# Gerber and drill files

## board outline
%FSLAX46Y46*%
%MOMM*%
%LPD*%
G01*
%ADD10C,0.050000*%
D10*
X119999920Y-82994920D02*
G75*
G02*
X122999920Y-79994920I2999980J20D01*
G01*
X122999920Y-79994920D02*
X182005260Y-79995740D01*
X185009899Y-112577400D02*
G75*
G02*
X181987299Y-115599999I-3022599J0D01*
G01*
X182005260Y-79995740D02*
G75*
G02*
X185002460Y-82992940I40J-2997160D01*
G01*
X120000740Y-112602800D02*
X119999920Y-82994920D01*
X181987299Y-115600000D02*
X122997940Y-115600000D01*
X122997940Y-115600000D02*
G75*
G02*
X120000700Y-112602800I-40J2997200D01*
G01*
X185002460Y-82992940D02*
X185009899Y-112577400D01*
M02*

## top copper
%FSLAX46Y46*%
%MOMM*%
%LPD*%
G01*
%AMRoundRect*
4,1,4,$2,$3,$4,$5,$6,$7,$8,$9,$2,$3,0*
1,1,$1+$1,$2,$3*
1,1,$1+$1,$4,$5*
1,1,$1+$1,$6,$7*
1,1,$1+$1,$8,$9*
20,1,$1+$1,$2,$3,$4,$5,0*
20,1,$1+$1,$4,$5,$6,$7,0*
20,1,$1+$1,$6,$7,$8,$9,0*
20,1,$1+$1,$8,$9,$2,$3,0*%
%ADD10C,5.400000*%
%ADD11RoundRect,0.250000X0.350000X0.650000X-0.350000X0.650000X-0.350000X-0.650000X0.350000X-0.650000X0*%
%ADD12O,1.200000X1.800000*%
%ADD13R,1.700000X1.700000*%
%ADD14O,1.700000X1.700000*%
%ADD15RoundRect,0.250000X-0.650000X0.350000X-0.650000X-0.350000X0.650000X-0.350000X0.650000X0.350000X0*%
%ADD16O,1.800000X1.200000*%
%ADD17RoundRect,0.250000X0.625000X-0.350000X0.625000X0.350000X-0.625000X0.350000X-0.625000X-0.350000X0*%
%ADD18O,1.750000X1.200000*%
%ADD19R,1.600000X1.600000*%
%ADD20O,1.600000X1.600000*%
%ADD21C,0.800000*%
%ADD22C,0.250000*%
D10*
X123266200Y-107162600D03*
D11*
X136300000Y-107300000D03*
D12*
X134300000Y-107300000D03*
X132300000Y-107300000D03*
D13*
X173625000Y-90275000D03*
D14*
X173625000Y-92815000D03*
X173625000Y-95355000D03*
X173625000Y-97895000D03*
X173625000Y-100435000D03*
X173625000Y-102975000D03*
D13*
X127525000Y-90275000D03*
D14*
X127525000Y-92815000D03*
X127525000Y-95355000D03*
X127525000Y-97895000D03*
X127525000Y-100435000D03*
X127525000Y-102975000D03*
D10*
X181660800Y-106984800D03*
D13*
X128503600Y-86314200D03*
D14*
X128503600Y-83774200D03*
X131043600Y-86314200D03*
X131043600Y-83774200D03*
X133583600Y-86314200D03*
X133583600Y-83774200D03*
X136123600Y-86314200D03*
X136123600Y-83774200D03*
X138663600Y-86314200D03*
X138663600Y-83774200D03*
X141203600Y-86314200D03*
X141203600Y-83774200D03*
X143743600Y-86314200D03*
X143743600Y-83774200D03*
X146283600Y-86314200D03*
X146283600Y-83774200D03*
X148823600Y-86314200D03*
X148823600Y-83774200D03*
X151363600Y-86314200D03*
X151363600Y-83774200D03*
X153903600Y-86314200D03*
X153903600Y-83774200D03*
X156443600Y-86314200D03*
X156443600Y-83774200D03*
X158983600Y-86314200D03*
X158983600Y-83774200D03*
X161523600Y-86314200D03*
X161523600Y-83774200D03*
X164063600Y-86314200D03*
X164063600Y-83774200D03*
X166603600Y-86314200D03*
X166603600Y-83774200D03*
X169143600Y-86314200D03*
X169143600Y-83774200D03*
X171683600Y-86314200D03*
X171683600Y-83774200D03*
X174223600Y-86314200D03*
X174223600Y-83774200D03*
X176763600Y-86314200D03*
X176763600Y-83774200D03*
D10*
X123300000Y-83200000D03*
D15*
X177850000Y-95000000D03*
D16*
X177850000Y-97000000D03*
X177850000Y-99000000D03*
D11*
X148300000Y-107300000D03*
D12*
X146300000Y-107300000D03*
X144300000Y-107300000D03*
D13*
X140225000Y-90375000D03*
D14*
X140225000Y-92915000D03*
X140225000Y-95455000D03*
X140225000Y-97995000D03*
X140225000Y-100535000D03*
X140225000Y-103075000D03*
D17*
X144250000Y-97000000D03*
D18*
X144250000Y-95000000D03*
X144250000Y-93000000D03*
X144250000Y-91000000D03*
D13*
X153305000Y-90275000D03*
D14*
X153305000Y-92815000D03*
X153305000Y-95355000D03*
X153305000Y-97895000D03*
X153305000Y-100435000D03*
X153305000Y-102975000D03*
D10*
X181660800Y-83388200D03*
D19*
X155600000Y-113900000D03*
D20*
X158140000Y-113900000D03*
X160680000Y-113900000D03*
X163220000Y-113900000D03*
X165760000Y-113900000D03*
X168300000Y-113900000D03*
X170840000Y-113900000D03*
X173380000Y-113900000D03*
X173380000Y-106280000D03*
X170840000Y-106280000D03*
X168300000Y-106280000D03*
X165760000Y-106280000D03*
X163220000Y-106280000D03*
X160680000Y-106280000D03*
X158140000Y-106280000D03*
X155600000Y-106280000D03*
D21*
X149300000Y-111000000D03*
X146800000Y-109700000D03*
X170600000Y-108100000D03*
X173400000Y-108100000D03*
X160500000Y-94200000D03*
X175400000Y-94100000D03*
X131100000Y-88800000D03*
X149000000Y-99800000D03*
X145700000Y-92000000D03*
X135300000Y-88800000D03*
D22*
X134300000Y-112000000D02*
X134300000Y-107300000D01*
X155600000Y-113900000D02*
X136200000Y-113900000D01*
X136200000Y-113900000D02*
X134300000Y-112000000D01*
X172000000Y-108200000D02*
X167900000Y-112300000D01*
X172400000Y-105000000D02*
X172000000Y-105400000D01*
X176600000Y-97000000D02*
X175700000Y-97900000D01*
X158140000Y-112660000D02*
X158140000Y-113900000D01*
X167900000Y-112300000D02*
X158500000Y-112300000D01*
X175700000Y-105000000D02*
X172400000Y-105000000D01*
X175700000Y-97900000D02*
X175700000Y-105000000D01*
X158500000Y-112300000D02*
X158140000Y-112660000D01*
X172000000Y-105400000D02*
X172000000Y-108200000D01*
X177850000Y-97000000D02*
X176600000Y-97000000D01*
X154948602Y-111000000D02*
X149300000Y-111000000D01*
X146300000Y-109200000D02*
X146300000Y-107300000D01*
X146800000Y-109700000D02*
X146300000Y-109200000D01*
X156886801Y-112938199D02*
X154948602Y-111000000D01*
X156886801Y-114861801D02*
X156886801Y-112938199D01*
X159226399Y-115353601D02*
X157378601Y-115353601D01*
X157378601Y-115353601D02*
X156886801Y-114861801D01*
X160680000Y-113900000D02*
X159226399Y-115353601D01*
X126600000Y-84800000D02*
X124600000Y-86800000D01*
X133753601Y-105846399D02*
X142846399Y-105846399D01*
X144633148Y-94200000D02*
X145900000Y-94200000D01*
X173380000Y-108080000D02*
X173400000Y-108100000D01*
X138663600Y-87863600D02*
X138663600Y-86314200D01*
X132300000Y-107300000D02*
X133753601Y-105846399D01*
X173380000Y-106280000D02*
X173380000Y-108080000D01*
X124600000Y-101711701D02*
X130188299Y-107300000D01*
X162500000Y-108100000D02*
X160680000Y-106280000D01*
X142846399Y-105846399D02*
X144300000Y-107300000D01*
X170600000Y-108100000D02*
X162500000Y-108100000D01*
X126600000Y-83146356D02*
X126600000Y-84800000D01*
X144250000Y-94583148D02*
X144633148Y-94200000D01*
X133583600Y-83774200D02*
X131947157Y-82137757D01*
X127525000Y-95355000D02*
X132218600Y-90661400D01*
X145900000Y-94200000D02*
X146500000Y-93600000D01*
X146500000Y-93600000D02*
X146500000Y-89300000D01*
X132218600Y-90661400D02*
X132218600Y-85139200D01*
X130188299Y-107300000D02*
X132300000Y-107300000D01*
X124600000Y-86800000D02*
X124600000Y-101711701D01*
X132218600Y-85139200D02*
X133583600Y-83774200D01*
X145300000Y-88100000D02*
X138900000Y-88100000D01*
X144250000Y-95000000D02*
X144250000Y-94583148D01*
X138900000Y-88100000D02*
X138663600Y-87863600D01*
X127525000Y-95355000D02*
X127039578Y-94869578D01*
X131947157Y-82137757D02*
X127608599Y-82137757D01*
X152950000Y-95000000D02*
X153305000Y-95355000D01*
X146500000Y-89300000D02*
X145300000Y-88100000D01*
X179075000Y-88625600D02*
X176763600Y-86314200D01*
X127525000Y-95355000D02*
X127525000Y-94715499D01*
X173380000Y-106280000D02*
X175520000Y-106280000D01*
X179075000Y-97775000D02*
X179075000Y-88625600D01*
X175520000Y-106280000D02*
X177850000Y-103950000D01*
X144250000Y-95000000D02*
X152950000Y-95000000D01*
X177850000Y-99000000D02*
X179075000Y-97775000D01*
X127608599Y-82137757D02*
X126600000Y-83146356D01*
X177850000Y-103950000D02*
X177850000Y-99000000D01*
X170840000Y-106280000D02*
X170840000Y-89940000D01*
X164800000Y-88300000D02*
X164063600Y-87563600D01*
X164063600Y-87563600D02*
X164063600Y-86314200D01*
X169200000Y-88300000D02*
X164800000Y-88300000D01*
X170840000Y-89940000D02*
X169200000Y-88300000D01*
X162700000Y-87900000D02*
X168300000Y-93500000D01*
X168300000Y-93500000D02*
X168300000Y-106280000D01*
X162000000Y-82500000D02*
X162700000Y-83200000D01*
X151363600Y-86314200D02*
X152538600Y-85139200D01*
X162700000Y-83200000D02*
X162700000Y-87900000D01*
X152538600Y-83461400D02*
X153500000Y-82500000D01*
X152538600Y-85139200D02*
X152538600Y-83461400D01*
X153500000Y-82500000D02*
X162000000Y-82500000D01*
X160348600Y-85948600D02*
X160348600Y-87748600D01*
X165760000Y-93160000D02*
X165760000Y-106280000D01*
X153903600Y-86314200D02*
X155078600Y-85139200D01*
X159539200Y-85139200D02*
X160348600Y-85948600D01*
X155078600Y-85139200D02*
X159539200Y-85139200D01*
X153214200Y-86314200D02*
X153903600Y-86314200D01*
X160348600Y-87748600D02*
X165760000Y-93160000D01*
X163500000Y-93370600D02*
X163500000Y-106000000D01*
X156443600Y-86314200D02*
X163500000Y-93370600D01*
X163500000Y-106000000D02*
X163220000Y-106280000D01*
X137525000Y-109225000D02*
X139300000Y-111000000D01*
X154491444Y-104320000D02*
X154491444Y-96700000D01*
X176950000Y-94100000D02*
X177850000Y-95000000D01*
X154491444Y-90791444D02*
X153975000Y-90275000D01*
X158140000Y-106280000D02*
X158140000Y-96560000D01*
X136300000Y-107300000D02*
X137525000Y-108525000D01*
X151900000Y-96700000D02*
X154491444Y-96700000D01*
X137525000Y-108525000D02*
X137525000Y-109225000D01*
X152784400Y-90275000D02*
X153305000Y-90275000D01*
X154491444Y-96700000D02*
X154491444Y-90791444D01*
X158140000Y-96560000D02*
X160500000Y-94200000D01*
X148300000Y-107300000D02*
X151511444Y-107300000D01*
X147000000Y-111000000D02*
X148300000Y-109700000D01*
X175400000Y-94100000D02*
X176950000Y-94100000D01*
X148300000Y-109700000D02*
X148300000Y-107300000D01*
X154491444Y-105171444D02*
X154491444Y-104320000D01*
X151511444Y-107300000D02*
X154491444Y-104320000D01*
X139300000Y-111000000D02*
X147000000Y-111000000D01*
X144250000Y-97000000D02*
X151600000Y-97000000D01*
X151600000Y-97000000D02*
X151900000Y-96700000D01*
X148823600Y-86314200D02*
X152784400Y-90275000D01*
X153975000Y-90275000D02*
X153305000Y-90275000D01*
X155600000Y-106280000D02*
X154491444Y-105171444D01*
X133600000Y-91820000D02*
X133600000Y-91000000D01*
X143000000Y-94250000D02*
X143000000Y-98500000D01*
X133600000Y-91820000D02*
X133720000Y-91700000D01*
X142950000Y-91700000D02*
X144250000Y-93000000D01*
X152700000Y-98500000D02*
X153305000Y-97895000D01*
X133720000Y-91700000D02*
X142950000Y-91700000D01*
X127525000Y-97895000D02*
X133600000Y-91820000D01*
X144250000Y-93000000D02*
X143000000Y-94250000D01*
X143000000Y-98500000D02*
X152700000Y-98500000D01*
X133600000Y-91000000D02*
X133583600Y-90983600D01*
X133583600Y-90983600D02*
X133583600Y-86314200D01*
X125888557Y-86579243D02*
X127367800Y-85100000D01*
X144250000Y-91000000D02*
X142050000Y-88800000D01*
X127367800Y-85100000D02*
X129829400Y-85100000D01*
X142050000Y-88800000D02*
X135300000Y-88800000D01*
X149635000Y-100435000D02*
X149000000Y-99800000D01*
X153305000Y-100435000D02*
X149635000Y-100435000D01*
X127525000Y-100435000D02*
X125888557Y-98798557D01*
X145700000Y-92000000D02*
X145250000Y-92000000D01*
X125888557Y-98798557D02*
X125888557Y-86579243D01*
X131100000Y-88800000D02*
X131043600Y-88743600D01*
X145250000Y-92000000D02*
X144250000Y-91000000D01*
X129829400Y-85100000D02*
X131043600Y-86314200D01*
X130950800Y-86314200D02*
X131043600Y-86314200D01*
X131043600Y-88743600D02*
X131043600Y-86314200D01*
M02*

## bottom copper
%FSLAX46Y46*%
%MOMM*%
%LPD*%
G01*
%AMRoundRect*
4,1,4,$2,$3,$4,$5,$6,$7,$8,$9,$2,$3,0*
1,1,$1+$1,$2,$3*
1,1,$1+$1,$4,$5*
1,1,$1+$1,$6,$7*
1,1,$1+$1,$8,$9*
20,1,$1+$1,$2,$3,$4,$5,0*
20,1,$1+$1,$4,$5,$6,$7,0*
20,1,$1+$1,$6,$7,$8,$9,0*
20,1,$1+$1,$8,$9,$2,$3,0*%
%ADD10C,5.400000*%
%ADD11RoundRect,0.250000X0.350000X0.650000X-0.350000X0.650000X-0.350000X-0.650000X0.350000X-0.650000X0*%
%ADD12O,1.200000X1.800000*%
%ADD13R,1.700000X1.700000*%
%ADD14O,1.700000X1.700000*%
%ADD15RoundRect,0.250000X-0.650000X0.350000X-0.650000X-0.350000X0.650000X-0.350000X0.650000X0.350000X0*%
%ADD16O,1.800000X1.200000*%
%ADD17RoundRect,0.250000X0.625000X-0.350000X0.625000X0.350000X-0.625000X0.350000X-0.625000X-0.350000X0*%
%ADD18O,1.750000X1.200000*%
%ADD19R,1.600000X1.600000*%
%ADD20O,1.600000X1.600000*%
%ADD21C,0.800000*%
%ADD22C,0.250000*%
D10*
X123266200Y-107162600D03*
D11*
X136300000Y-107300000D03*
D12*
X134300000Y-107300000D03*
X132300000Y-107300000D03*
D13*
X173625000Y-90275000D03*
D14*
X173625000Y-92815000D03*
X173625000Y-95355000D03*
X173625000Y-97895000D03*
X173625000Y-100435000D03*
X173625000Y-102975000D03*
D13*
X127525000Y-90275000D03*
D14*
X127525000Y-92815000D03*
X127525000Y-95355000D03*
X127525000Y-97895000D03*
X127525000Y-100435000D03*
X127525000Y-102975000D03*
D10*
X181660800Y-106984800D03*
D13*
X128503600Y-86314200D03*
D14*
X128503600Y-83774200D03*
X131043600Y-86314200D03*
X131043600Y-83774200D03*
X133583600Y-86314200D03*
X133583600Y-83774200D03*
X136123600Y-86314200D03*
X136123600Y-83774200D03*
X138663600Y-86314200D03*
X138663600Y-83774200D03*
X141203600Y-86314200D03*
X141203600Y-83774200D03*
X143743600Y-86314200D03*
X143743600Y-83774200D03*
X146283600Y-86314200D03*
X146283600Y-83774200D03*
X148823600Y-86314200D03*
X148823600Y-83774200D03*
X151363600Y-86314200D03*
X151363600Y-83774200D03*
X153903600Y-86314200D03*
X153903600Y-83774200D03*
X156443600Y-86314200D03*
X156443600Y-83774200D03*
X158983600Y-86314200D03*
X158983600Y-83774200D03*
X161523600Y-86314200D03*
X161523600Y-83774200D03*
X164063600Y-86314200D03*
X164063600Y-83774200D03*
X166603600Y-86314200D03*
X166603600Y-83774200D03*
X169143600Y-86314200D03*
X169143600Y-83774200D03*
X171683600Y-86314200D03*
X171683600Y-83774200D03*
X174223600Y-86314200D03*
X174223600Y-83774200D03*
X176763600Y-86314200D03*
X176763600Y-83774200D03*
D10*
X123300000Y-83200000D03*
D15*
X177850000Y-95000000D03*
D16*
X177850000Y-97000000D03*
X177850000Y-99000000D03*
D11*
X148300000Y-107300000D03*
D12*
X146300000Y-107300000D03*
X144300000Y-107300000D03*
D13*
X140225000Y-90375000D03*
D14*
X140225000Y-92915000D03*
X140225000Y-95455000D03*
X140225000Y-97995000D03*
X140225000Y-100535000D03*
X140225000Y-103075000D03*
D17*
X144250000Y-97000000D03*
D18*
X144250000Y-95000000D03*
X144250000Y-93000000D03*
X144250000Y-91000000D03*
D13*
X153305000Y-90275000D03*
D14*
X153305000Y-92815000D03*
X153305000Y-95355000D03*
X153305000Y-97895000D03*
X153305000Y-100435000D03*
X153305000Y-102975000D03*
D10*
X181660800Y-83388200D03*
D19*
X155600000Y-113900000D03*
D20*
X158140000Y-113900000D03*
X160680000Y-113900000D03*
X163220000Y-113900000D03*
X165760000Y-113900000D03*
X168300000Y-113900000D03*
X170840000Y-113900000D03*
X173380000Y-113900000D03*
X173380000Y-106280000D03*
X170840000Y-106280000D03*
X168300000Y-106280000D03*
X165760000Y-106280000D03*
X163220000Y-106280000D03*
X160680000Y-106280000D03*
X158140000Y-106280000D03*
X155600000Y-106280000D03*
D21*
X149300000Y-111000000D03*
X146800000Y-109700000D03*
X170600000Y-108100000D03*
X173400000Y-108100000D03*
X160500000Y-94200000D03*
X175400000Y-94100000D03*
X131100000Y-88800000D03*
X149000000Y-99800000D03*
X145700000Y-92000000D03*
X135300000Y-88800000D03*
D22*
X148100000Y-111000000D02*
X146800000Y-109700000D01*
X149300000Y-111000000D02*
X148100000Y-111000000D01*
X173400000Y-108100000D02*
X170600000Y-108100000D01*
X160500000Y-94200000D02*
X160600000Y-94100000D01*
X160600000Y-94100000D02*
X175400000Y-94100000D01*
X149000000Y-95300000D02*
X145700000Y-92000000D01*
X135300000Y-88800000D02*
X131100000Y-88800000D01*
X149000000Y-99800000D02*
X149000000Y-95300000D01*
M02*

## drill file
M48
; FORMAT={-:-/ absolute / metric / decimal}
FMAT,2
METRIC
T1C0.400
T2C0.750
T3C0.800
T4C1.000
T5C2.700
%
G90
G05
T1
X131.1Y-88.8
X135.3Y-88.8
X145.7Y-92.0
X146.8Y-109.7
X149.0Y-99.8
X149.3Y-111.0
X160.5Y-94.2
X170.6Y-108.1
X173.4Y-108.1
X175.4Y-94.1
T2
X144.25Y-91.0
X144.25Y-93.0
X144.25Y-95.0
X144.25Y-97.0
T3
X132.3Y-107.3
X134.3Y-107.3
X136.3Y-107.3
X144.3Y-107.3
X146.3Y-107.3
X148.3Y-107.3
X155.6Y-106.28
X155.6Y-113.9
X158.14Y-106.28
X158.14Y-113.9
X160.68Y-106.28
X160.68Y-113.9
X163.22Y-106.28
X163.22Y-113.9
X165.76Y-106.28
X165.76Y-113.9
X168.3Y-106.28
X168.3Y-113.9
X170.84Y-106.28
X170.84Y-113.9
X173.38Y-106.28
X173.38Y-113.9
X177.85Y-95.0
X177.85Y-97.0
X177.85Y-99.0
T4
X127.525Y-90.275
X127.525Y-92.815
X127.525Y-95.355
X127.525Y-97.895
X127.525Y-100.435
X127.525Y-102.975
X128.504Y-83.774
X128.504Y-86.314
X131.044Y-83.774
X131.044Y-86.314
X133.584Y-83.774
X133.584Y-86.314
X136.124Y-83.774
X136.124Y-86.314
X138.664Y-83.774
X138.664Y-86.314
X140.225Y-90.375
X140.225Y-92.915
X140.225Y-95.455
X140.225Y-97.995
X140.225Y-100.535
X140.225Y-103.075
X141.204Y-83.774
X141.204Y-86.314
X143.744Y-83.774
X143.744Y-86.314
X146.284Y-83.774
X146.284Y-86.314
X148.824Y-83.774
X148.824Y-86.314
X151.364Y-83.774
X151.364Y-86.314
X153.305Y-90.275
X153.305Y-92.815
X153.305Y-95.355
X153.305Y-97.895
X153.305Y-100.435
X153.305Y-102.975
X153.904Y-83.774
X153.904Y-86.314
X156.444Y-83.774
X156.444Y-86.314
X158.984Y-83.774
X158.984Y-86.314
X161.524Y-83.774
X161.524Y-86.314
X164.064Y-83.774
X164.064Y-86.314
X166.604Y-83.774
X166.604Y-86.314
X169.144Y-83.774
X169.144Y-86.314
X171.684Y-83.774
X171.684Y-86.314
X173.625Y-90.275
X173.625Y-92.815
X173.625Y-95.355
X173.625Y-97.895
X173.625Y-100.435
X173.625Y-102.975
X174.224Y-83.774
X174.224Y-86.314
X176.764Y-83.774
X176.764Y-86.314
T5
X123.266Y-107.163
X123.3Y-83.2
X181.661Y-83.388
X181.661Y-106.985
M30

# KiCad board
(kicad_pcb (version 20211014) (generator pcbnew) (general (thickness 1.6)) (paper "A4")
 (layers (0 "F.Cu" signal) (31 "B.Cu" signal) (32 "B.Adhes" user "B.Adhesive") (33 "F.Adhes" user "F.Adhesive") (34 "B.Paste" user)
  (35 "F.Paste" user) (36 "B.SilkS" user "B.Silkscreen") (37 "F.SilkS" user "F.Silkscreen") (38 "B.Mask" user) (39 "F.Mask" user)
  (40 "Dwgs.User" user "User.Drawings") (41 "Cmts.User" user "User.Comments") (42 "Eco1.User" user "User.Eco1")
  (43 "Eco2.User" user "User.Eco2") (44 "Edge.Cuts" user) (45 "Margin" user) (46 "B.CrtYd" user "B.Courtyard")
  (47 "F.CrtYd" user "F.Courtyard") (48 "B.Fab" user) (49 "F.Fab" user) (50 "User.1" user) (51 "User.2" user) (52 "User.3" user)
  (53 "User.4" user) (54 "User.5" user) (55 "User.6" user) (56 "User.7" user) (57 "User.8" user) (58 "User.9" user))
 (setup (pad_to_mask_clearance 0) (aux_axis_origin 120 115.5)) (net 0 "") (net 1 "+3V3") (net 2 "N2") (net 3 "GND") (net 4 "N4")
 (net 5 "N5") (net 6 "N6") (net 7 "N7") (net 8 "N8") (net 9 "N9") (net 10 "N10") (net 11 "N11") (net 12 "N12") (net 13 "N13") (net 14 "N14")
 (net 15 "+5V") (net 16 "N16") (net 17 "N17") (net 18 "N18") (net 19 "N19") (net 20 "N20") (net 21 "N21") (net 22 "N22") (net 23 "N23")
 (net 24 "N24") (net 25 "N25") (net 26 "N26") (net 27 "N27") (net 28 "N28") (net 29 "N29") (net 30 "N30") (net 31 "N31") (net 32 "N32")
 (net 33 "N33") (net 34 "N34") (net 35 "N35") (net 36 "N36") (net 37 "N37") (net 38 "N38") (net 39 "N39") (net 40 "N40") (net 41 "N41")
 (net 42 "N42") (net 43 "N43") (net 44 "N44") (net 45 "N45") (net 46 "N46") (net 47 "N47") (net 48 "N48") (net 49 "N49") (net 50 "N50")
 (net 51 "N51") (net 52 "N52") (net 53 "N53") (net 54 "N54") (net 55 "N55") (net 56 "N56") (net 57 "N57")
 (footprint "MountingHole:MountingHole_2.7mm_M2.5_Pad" (layer "F.Cu") (at 123.2662 107.1626)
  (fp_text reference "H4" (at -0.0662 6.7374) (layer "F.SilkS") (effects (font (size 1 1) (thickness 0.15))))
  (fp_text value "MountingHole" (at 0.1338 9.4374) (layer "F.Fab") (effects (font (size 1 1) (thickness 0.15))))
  (pad "1" thru_hole circle (at 0 0) (size 5.4 5.4) (drill 2.7) (layers *.Cu *.Mask)))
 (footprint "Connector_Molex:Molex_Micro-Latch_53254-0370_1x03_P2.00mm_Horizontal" (layer "F.Cu") (at 136.3 107.3 180)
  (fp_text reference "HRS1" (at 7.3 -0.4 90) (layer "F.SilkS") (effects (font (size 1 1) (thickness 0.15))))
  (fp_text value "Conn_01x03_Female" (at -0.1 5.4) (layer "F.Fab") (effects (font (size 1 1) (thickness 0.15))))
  (pad "1" thru_hole roundrect (at 0 0 180) (size 1.2 1.8) (drill 0.8) (layers *.Cu *.Mask) (roundrect_rratio 0.208333) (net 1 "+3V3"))
  (pad "2" thru_hole oval (at 2 0 180) (size 1.2 1.8) (drill 0.8) (layers *.Cu *.Mask) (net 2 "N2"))
  (pad "3" thru_hole oval (at 4 0 180) (size 1.2 1.8) (drill 0.8) (layers *.Cu *.Mask) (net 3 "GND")))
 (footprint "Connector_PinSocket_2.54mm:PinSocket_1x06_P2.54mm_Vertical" (layer "F.Cu") (at 173.625 90.275)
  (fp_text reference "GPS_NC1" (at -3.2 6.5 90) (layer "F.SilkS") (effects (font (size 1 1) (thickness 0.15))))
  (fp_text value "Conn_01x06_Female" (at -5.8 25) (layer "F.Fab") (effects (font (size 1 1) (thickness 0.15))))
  (pad "1" thru_hole rect (at 0 0) (size 1.7 1.7) (drill 1) (layers *.Cu *.Mask) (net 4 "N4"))
  (pad "2" thru_hole oval (at 0 2.54) (size 1.7 1.7) (drill 1) (layers *.Cu *.Mask) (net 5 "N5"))
  (pad "3" thru_hole oval (at 0 5.08) (size 1.7 1.7) (drill 1) (layers *.Cu *.Mask) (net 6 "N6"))
  (pad "4" thru_hole oval (at 0 7.62) (size 1.7 1.7) (drill 1) (layers *.Cu *.Mask) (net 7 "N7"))
  (pad "5" thru_hole oval (at 0 10.16) (size 1.7 1.7) (drill 1) (layers *.Cu *.Mask) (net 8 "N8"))
  (pad "6" thru_hole oval (at 0 12.7) (size 1.7 1.7) (drill 1) (layers *.Cu *.Mask) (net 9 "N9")))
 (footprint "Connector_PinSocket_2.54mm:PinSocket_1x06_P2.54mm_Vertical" (layer "F.Cu") (at 127.525 90.275)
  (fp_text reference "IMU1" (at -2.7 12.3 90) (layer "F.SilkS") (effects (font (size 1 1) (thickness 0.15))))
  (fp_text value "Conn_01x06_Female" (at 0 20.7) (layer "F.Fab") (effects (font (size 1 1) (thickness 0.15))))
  (pad "1" thru_hole rect (at 0 0) (size 1.7 1.7) (drill 1) (layers *.Cu *.Mask) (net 1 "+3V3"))
  (pad "2" thru_hole oval (at 0 2.54) (size 1.7 1.7) (drill 1) (layers *.Cu *.Mask) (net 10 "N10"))
  (pad "3" thru_hole oval (at 0 5.08) (size 1.7 1.7) (drill 1) (layers *.Cu *.Mask) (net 3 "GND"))
  (pad "4" thru_hole oval (at 0 7.62) (size 1.7 1.7) (drill 1) (layers *.Cu *.Mask) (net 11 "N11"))
  (pad "5" thru_hole oval (at 0 10.16) (size 1.7 1.7) (drill 1) (layers *.Cu *.Mask) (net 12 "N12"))
  (pad "6" thru_hole oval (at 0 12.7) (size 1.7 1.7) (drill 1) (layers *.Cu *.Mask) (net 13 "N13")))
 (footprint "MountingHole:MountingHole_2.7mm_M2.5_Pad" (layer "F.Cu") (at 181.6608 106.9848)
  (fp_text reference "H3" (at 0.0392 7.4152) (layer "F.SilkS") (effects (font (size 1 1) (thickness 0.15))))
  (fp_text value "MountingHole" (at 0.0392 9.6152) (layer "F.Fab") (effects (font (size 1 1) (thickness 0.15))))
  (pad "1" thru_hole circle (at 0 0) (size 5.4 5.4) (drill 2.7) (layers *.Cu *.Mask)))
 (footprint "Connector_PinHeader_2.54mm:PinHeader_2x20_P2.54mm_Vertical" (layer "F.Cu") (at 128.5036 86.3142 90)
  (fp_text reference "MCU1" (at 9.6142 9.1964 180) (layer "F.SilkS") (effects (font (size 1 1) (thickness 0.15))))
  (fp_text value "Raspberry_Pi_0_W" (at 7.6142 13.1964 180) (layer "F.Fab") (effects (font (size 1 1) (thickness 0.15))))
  (pad "1" thru_hole rect (at 0 0 90) (size 1.7 1.7) (drill 1) (layers *.Cu *.Mask) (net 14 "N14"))
  (pad "2" thru_hole oval (at 2.54 0 90) (size 1.7 1.7) (drill 1) (layers *.Cu *.Mask) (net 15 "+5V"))
  (pad "3" thru_hole oval (at 0 2.54 90) (size 1.7 1.7) (drill 1) (layers *.Cu *.Mask) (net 12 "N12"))
  (pad "4" thru_hole oval (at 2.54 2.54 90) (size 1.7 1.7) (drill 1) (layers *.Cu *.Mask) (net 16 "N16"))
  (pad "5" thru_hole oval (at 0 5.08 90) (size 1.7 1.7) (drill 1) (layers *.Cu *.Mask) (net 11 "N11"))
  (pad "6" thru_hole oval (at 2.54 5.08 90) (size 1.7 1.7) (drill 1) (layers *.Cu *.Mask) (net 3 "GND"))
  (pad "7" thru_hole oval (at 0 7.62 90) (size 1.7 1.7) (drill 1) (layers *.Cu *.Mask) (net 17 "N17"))
  (pad "8" thru_hole oval (at 2.54 7.62 90) (size 1.7 1.7) (drill 1) (layers *.Cu *.Mask) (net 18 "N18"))
  (pad "9" thru_hole oval (at 0 10.16 90) (size 1.7 1.7) (drill 1) (layers *.Cu *.Mask) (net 3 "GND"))
  (pad "10" thru_hole oval (at 2.54 10.16 90) (size 1.7 1.7) (drill 1) (layers *.Cu *.Mask) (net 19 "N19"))
  (pad "11" thru_hole oval (at 0 12.7 90) (size 1.7 1.7) (drill 1) (layers *.Cu *.Mask) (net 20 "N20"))
  (pad "12" thru_hole oval (at 2.54 12.7 90) (size 1.7 1.7) (drill 1) (layers *.Cu *.Mask) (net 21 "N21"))
  (pad "13" thru_hole oval (at 0 15.24 90) (size 1.7 1.7) (drill 1) (layers *.Cu *.Mask) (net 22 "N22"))
  (pad "14" thru_hole oval (at 2.54 15.24 90) (size 1.7 1.7) (drill 1) (layers *.Cu *.Mask) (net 3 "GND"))
  (pad "15" thru_hole oval (at 0 17.78 90) (size 1.7 1.7) (drill 1) (layers *.Cu *.Mask) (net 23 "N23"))
  (pad "16" thru_hole oval (at 2.54 17.78 90) (size 1.7 1.7) (drill 1) (layers *.Cu *.Mask) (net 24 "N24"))
  (pad "17" thru_hole oval (at 0 20.32 90) (size 1.7 1.7) (drill 1) (layers *.Cu *.Mask) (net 1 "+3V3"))
  (pad "18" thru_hole oval (at 2.54 20.32 90) (size 1.7 1.7) (drill 1) (layers *.Cu *.Mask) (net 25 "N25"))
  (pad "19" thru_hole oval (at 0 22.86 90) (size 1.7 1.7) (drill 1) (layers *.Cu *.Mask) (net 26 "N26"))
  (pad "20" thru_hole oval (at 2.54 22.86 90) (size 1.7 1.7) (drill 1) (layers *.Cu *.Mask) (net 3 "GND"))
  (pad "21" thru_hole oval (at 0 25.4 90) (size 1.7 1.7) (drill 1) (layers *.Cu *.Mask) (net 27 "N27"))
  (pad "22" thru_hole oval (at 2.54 25.4 90) (size 1.7 1.7) (drill 1) (layers *.Cu *.Mask) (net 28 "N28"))
  (pad "23" thru_hole oval (at 0 27.94 90) (size 1.7 1.7) (drill 1) (layers *.Cu *.Mask) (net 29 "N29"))
  (pad "24" thru_hole oval (at 2.54 27.94 90) (size 1.7 1.7) (drill 1) (layers *.Cu *.Mask) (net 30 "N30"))
  (pad "25" thru_hole oval (at 0 30.48 90) (size 1.7 1.7) (drill 1) (layers *.Cu *.Mask) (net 3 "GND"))
  (pad "26" thru_hole oval (at 2.54 30.48 90) (size 1.7 1.7) (drill 1) (layers *.Cu *.Mask) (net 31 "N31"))
  (pad "27" thru_hole oval (at 0 33.02 90) (size 1.7 1.7) (drill 1) (layers *.Cu *.Mask) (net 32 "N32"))
  (pad "28" thru_hole oval (at 2.54 33.02 90) (size 1.7 1.7) (drill 1) (layers *.Cu *.Mask) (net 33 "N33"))
  (pad "29" thru_hole oval (at 0 35.56 90) (size 1.7 1.7) (drill 1) (layers *.Cu *.Mask) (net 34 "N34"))
  (pad "30" thru_hole oval (at 2.54 35.56 90) (size 1.7 1.7) (drill 1) (layers *.Cu *.Mask) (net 3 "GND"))
  (pad "31" thru_hole oval (at 0 38.1 90) (size 1.7 1.7) (drill 1) (layers *.Cu *.Mask) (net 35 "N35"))
  (pad "32" thru_hole oval (at 2.54 38.1 90) (size 1.7 1.7) (drill 1) (layers *.Cu *.Mask) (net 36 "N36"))
  (pad "33" thru_hole oval (at 0 40.64 90) (size 1.7 1.7) (drill 1) (layers *.Cu *.Mask) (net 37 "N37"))
  (pad "34" thru_hole oval (at 2.54 40.64 90) (size 1.7 1.7) (drill 1) (layers *.Cu *.Mask) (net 3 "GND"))
  (pad "35" thru_hole oval (at 0 43.18 90) (size 1.7 1.7) (drill 1) (layers *.Cu *.Mask) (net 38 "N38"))
  (pad "36" thru_hole oval (at 2.54 43.18 90) (size 1.7 1.7) (drill 1) (layers *.Cu *.Mask) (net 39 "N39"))
  (pad "37" thru_hole oval (at 0 45.72 90) (size 1.7 1.7) (drill 1) (layers *.Cu *.Mask) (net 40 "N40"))
  (pad "38" thru_hole oval (at 2.54 45.72 90) (size 1.7 1.7) (drill 1) (layers *.Cu *.Mask) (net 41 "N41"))
  (pad "39" thru_hole oval (at 0 48.26 90) (size 1.7 1.7) (drill 1) (layers *.Cu *.Mask) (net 3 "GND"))
  (pad "40" thru_hole oval (at 2.54 48.26 90) (size 1.7 1.7) (drill 1) (layers *.Cu *.Mask) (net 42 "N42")))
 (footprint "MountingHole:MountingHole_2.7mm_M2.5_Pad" (layer "F.Cu") (at 123.3 83.2)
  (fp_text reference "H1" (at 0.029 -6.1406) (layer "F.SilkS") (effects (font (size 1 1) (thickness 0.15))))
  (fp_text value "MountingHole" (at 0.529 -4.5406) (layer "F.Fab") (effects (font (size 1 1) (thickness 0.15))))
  (pad "1" thru_hole circle (at 0 0) (size 5.4 5.4) (drill 2.7) (layers *.Cu *.Mask)))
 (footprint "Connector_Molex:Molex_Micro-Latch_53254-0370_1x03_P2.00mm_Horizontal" (layer "F.Cu") (at 177.85 95 -90)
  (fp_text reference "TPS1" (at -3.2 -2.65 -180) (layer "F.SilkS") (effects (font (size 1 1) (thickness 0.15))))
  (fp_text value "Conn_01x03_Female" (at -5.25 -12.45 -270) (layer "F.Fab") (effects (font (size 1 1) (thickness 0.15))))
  (pad "1" thru_hole roundrect (at 0 0 270) (size 1.2 1.8) (drill 0.8) (layers *.Cu *.Mask) (roundrect_rratio 0.208333) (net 1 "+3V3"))
  (pad "2" thru_hole oval (at 2 0 270) (size 1.2 1.8) (drill 0.8) (layers *.Cu *.Mask) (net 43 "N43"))
  (pad "3" thru_hole oval (at 4 0 270) (size 1.2 1.8) (drill 0.8) (layers *.Cu *.Mask) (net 3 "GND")))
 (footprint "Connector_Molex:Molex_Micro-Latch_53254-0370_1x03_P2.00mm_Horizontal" (layer "F.Cu") (at 148.3 107.3 180)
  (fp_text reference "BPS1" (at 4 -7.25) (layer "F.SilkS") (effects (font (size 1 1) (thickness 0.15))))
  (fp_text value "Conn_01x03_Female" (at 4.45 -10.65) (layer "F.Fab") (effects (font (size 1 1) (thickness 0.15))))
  (pad "1" thru_hole roundrect (at 0 0 180) (size 1.2 1.8) (drill 0.8) (layers *.Cu *.Mask) (roundrect_rratio 0.208333) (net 1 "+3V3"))
  (pad "2" thru_hole oval (at 2 0 180) (size 1.2 1.8) (drill 0.8) (layers *.Cu *.Mask) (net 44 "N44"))
  (pad "3" thru_hole oval (at 4 0 180) (size 1.2 1.8) (drill 0.8) (layers *.Cu *.Mask) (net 3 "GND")))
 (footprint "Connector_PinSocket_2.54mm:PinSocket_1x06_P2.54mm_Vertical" (layer "F.Cu") (at 140.225 90.375)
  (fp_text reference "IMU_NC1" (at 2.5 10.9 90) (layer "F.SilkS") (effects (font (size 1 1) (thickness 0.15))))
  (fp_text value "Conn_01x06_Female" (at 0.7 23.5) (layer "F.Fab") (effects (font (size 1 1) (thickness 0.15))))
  (pad "1" thru_hole rect (at 0 0) (size 1.7 1.7) (drill 1) (layers *.Cu *.Mask) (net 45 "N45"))
  (pad "2" thru_hole oval (at 0 2.54) (size 1.7 1.7) (drill 1) (layers *.Cu *.Mask) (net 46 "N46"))
  (pad "3" thru_hole oval (at 0 5.08) (size 1.7 1.7) (drill 1) (layers *.Cu *.Mask) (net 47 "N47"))
  (pad "4" thru_hole oval (at 0 7.62) (size 1.7 1.7) (drill 1) (layers *.Cu *.Mask) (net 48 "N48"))
  (pad "5" thru_hole oval (at 0 10.16) (size 1.7 1.7) (drill 1) (layers *.Cu *.Mask) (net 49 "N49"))
  (pad "6" thru_hole oval (at 0 12.7) (size 1.7 1.7) (drill 1) (layers *.Cu *.Mask) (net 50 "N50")))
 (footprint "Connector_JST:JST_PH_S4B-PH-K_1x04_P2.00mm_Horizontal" (layer "F.Cu") (at 144.25 97 90)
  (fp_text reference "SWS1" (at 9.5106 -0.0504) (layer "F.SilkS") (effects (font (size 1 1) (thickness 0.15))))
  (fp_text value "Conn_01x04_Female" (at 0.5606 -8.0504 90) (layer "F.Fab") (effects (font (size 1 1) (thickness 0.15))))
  (pad "1" thru_hole roundrect (at 0 0 90) (size 1.2 1.75) (drill 0.75) (layers *.Cu *.Mask) (roundrect_rratio 0.208333) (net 1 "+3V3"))
  (pad "2" thru_hole oval (at 2 0 90) (size 1.2 1.75) (drill 0.75) (layers *.Cu *.Mask) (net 3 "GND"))
  (pad "3" thru_hole oval (at 4 0 90) (size 1.2 1.75) (drill 0.75) (layers *.Cu *.Mask) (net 11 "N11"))
  (pad "4" thru_hole oval (at 6 0 90) (size 1.2 1.75) (drill 0.75) (layers *.Cu *.Mask) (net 12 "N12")))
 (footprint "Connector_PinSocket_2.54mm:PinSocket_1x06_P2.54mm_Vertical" (layer "F.Cu") (at 153.305 90.275)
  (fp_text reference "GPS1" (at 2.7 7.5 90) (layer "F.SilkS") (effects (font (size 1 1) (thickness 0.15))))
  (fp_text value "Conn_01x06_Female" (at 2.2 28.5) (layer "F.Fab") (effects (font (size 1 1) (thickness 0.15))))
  (pad "1" thru_hole rect (at 0 0) (size 1.7 1.7) (drill 1) (layers *.Cu *.Mask) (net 1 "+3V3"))
  (pad "2" thru_hole oval (at 0 2.54) (size 1.7 1.7) (drill 1) (layers *.Cu *.Mask) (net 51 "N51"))
  (pad "3" thru_hole oval (at 0 5.08) (size 1.7 1.7) (drill 1) (layers *.Cu *.Mask) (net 3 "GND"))
  (pad "4" thru_hole oval (at 0 7.62) (size 1.7 1.7) (drill 1) (layers *.Cu *.Mask) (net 11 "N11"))
  (pad "5" thru_hole oval (at 0 10.16) (size 1.7 1.7) (drill 1) (layers *.Cu *.Mask) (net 12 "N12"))
  (pad "6" thru_hole oval (at 0 12.7) (size 1.7 1.7) (drill 1) (layers *.Cu *.Mask) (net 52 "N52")))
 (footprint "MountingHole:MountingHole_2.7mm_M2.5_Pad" (layer "F.Cu") (at 181.6608 83.3882)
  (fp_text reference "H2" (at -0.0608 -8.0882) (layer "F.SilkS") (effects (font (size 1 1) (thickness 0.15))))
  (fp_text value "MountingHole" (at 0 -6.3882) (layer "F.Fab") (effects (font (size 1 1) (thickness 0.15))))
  (pad "1" thru_hole circle (at 0 0) (size 5.4 5.4) (drill 2.7) (layers *.Cu *.Mask)))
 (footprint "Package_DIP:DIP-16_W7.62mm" (layer "F.Cu") (at 155.6 113.9 90)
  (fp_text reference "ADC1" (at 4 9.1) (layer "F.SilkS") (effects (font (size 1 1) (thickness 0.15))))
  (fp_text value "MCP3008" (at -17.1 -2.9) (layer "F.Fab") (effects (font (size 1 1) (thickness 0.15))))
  (pad "1" thru_hole rect (at 0 0 90) (size 1.6 1.6) (drill 0.8) (layers *.Cu *.Mask) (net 2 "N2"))
  (pad "2" thru_hole oval (at 0 2.54 90) (size 1.6 1.6) (drill 0.8) (layers *.Cu *.Mask) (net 43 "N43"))
  (pad "3" thru_hole oval (at 0 5.08 90) (size 1.6 1.6) (drill 0.8) (layers *.Cu *.Mask) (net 44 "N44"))
  (pad "4" thru_hole oval (at 0 7.62 90) (size 1.6 1.6) (drill 0.8) (layers *.Cu *.Mask) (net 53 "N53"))
  (pad "5" thru_hole oval (at 0 10.16 90) (size 1.6 1.6) (drill 0.8) (layers *.Cu *.Mask) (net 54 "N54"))
  (pad "6" thru_hole oval (at 0 12.7 90) (size 1.6 1.6) (drill 0.8) (layers *.Cu *.Mask) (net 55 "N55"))
  (pad "7" thru_hole oval (at 0 15.24 90) (size 1.6 1.6) (drill 0.8) (layers *.Cu *.Mask) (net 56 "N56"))
  (pad "8" thru_hole oval (at 0 17.78 90) (size 1.6 1.6) (drill 0.8) (layers *.Cu *.Mask) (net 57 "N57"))
  (pad "9" thru_hole oval (at 7.62 17.78 90) (size 1.6 1.6) (drill 0.8) (layers *.Cu *.Mask) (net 3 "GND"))
  (pad "10" thru_hole oval (at 7.62 15.24 90) (size 1.6 1.6) (drill 0.8) (layers *.Cu *.Mask) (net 34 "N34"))
  (pad "11" thru_hole oval (at 7.62 12.7 90) (size 1.6 1.6) (drill 0.8) (layers *.Cu *.Mask) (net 26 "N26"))
  (pad "12" thru_hole oval (at 7.62 10.16 90) (size 1.6 1.6) (drill 0.8) (layers *.Cu *.Mask) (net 27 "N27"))
  (pad "13" thru_hole oval (at 7.62 7.62 90) (size 1.6 1.6) (drill 0.8) (layers *.Cu *.Mask) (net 29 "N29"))
  (pad "14" thru_hole oval (at 7.62 5.08 90) (size 1.6 1.6) (drill 0.8) (layers *.Cu *.Mask) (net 3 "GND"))
  (pad "15" thru_hole oval (at 7.62 2.54 90) (size 1.6 1.6) (drill 0.8) (layers *.Cu *.Mask) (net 1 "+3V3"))
  (pad "16" thru_hole oval (at 7.62 0 90) (size 1.6 1.6) (drill 0.8) (layers *.Cu *.Mask) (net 1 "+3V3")))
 (gr_arc (start 119.99992 82.99492) (mid 120.878594 80.873594) (end 122.99992 79.99492) (layer "Edge.Cuts") (width 0.05))
 (gr_line (start 122.99992 79.99492) (end 182.00526 79.99574) (layer "Edge.Cuts") (width 0.05))
 (gr_arc (start 185.009899 112.5774) (mid 184.1246 114.714701) (end 181.987299 115.6) (layer "Edge.Cuts") (width 0.05))
 (gr_arc (start 182.00526 79.99574) (mid 184.1246 80.8736) (end 185.00246 82.99294) (layer "Edge.Cuts") (width 0.05))
 (gr_line (start 120.00074 112.6028) (end 119.99992 82.99492) (layer "Edge.Cuts") (width 0.05))
 (gr_line (start 181.987299 115.6) (end 122.99794 115.6) (layer "Edge.Cuts") (width 0.05))
 (gr_arc (start 122.99794 115.6) (mid 120.878588 114.722152) (end 120.00074 112.6028) (layer "Edge.Cuts") (width 0.05))
 (gr_line (start 185.00246 82.99294) (end 185.009899 112.5774) (layer "Edge.Cuts") (width 0.05))
 (segment (start 134.3 112) (end 134.3 107.3) (width 0.25) (layer "F.Cu") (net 2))
 (segment (start 155.6 113.9) (end 136.2 113.9) (width 0.25) (layer "F.Cu") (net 2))
 (segment (start 136.2 113.9) (end 134.3 112) (width 0.25) (layer "F.Cu") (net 2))
 (segment (start 172 108.2) (end 167.9 112.3) (width 0.25) (layer "F.Cu") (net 43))
 (segment (start 172.4 105) (end 172 105.4) (width 0.25) (layer "F.Cu") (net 43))
 (segment (start 176.6 97) (end 175.7 97.9) (width 0.25) (layer "F.Cu") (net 43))
 (segment (start 158.14 112.66) (end 158.14 113.9) (width 0.25) (layer "F.Cu") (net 43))
 (segment (start 167.9 112.3) (end 158.5 112.3) (width 0.25) (layer "F.Cu") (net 43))
 (segment (start 175.7 105) (end 172.4 105) (width 0.25) (layer "F.Cu") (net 43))
 (segment (start 175.7 97.9) (end 175.7 105) (width 0.25) (layer "F.Cu") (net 43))
 (segment (start 158.5 112.3) (end 158.14 112.66) (width 0.25) (layer "F.Cu") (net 43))
 (segment (start 172 105.4) (end 172 108.2) (width 0.25) (layer "F.Cu") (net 43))
 (segment (start 177.85 97) (end 176.6 97) (width 0.25) (layer "F.Cu") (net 43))
 (segment (start 154.948602 111) (end 149.3 111) (width 0.25) (layer "F.Cu") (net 44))
 (segment (start 146.3 109.2) (end 146.3 107.3) (width 0.25) (layer "F.Cu") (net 44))
 (segment (start 146.8 109.7) (end 146.3 109.2) (width 0.25) (layer "F.Cu") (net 44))
 (segment (start 156.886801 112.938199) (end 154.948602 111) (width 0.25) (layer "F.Cu") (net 44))
 (segment (start 156.886801 114.861801) (end 156.886801 112.938199) (width 0.25) (layer "F.Cu") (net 44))
 (segment (start 159.226399 115.353601) (end 157.378601 115.353601) (width 0.25) (layer "F.Cu") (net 44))
 (segment (start 157.378601 115.353601) (end 156.886801 114.861801) (width 0.25) (layer "F.Cu") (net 44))
 (segment (start 160.68 113.9) (end 159.226399 115.353601) (width 0.25) (layer "F.Cu") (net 44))
 (via (at 149.3 111) (size 0.8) (drill 0.4) (layers "F.Cu" "B.Cu") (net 44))
 (via (at 146.8 109.7) (size 0.8) (drill 0.4) (layers "F.Cu" "B.Cu") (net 44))
 (segment (start 148.1 111) (end 146.8 109.7) (width 0.25) (layer "B.Cu") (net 44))
 (segment (start 149.3 111) (end 148.1 111) (width 0.25) (layer "B.Cu") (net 44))
 (segment (start 126.6 84.8) (end 124.6 86.8) (width 0.25) (layer "F.Cu") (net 3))
 (segment (start 133.753601 105.846399) (end 142.846399 105.846399) (width 0.25) (layer "F.Cu") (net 3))
 (segment (start 144.633148 94.2) (end 145.9 94.2) (width 0.25) (layer "F.Cu") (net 3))
 (segment (start 173.38 108.08) (end 173.4 108.1) (width 0.25) (layer "F.Cu") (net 3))
 (segment (start 138.6636 87.8636) (end 138.6636 86.3142) (width 0.25) (layer "F.Cu") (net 3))
 (segment (start 132.3 107.3) (end 133.753601 105.846399) (width 0.25) (layer "F.Cu") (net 3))
 (segment (start 173.38 106.28) (end 173.38 108.08) (width 0.25) (layer "F.Cu") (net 3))
 (segment (start 124.6 101.711701) (end 130.188299 107.3) (width 0.25) (layer "F.Cu") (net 3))
 (segment (start 162.5 108.1) (end 160.68 106.28) (width 0.25) (layer "F.Cu") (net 3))
 (segment (start 142.846399 105.846399) (end 144.3 107.3) (width 0.25) (layer "F.Cu") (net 3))
 (segment (start 170.6 108.1) (end 162.5 108.1) (width 0.25) (layer "F.Cu") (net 3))
 (segment (start 126.6 83.146356) (end 126.6 84.8) (width 0.25) (layer "F.Cu") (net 3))
 (segment (start 144.25 94.583148) (end 144.633148 94.2) (width 0.25) (layer "F.Cu") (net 3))
 (segment (start 133.5836 83.7742) (end 131.947157 82.137757) (width 0.25) (layer "F.Cu") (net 3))
 (segment (start 127.525 95.355) (end 132.2186 90.6614) (width 0.25) (layer "F.Cu") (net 3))
 (segment (start 145.9 94.2) (end 146.5 93.6) (width 0.25) (layer "F.Cu") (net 3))
 (segment (start 146.5 93.6) (end 146.5 89.3) (width 0.25) (layer "F.Cu") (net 3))
 (segment (start 132.2186 90.6614) (end 132.2186 85.1392) (width 0.25) (layer "F.Cu") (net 3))
 (segment (start 130.188299 107.3) (end 132.3 107.3) (width 0.25) (layer "F.Cu") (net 3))
 (segment (start 124.6 86.8) (end 124.6 101.711701) (width 0.25) (layer "F.Cu") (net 3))
 (segment (start 132.2186 85.1392) (end 133.5836 83.7742) (width 0.25) (layer "F.Cu") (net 3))
 (segment (start 145.3 88.1) (end 138.9 88.1) (width 0.25) (layer "F.Cu") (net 3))
 (segment (start 144.25 95) (end 144.25 94.583148) (width 0.25) (layer "F.Cu") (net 3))
 (segment (start 138.9 88.1) (end 138.6636 87.8636) (width 0.25) (layer "F.Cu") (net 3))
 (segment (start 127.525 95.355) (end 127.039578 94.869578) (width 0.25) (layer "F.Cu") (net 3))
 (segment (start 131.947157 82.137757) (end 127.608599 82.137757) (width 0.25) (layer "F.Cu") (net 3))
 (segment (start 152.95 95) (end 153.305 95.355) (width 0.25) (layer "F.Cu") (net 3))
 (segment (start 146.5 89.3) (end 145.3 88.1) (width 0.25) (layer "F.Cu") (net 3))
 (segment (start 179.075 88.6256) (end 176.7636 86.3142) (width 0.25) (layer "F.Cu") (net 3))
 (segment (start 127.525 95.355) (end 127.525 94.715499) (width 0.25) (layer "F.Cu") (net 3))
 (segment (start 173.38 106.28) (end 175.52 106.28) (width 0.25) (layer "F.Cu") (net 3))
 (segment (start 179.075 97.775) (end 179.075 88.6256) (width 0.25) (layer "F.Cu") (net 3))
 (segment (start 175.52 106.28) (end 177.85 103.95) (width 0.25) (layer "F.Cu") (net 3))
 (segment (start 144.25 95) (end 152.95 95) (width 0.25) (layer "F.Cu") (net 3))
 (segment (start 177.85 99) (end 179.075 97.775) (width 0.25) (layer "F.Cu") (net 3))
 (segment (start 127.608599 82.137757) (end 126.6 83.146356) (width 0.25) (layer "F.Cu") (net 3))
 (segment (start 177.85 103.95) (end 177.85 99) (width 0.25) (layer "F.Cu") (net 3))
 (via (at 170.6 108.1) (size 0.8) (drill 0.4) (layers "F.Cu" "B.Cu") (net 3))
 (via (at 173.4 108.1) (size 0.8) (drill 0.4) (layers "F.Cu" "B.Cu") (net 3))
 (segment (start 173.4 108.1) (end 170.6 108.1) (width 0.25) (layer "B.Cu") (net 3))
 (segment (start 170.84 106.28) (end 170.84 89.94) (width 0.25) (layer "F.Cu") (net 34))
 (segment (start 164.8 88.3) (end 164.0636 87.5636) (width 0.25) (layer "F.Cu") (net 34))
 (segment (start 164.0636 87.5636) (end 164.0636 86.3142) (width 0.25) (layer "F.Cu") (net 34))
 (segment (start 169.2 88.3) (end 164.8 88.3) (width 0.25) (layer "F.Cu") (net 34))
 (segment (start 170.84 89.94) (end 169.2 88.3) (width 0.25) (layer "F.Cu") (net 34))
 (segment (start 162.7 87.9) (end 168.3 93.5) (width 0.25) (layer "F.Cu") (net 26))
 (segment (start 168.3 93.5) (end 168.3 106.28) (width 0.25) (layer "F.Cu") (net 26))
 (segment (start 162 82.5) (end 162.7 83.2) (width 0.25) (layer "F.Cu") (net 26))
 (segment (start 151.3636 86.3142) (end 152.5386 85.1392) (width 0.25) (layer "F.Cu") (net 26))
 (segment (start 162.7 83.2) (end 162.7 87.9) (width 0.25) (layer "F.Cu") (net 26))
 (segment (start 152.5386 83.4614) (end 153.5 82.5) (width 0.25) (layer "F.Cu") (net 26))
 (segment (start 152.5386 85.1392) (end 152.5386 83.4614) (width 0.25) (layer "F.Cu") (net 26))
 (segment (start 153.5 82.5) (end 162 82.5) (width 0.25) (layer "F.Cu") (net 26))
 (segment (start 160.3486 85.9486) (end 160.3486 87.7486) (width 0.25) (layer "F.Cu") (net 27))
 (segment (start 165.76 93.16) (end 165.76 106.28) (width 0.25) (layer "F.Cu") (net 27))
 (segment (start 153.9036 86.3142) (end 155.0786 85.1392) (width 0.25) (layer "F.Cu") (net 27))
 (segment (start 159.5392 85.1392) (end 160.3486 85.9486) (width 0.25) (layer "F.Cu") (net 27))
 (segment (start 155.0786 85.1392) (end 159.5392 85.1392) (width 0.25) (layer "F.Cu") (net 27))
 (segment (start 153.2142 86.3142) (end 153.9036 86.3142) (width 0.25) (layer "F.Cu") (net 27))
 (segment (start 160.3486 87.7486) (end 165.76 93.16) (width 0.25) (layer "F.Cu") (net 27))
 (segment (start 163.5 93.3706) (end 163.5 106) (width 0.25) (layer "F.Cu") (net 29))
 (segment (start 156.4436 86.3142) (end 163.5 93.3706) (width 0.25) (layer "F.Cu") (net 29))
 (segment (start 163.5 106) (end 163.22 106.28) (width 0.25) (layer "F.Cu") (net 29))
 (segment (start 137.525 109.225) (end 139.3 111) (width 0.25) (layer "F.Cu") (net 1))
 (segment (start 154.491444 104.32) (end 154.491444 96.7) (width 0.25) (layer "F.Cu") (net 1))
 (segment (start 176.95 94.1) (end 177.85 95) (width 0.25) (layer "F.Cu") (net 1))
 (segment (start 154.491444 90.791444) (end 153.975 90.275) (width 0.25) (layer "F.Cu") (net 1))
 (segment (start 158.14 106.28) (end 158.14 96.56) (width 0.25) (layer "F.Cu") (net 1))
 (segment (start 136.3 107.3) (end 137.525 108.525) (width 0.25) (layer "F.Cu") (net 1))
 (segment (start 151.9 96.7) (end 154.491444 96.7) (width 0.25) (layer "F.Cu") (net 1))
 (segment (start 137.525 108.525) (end 137.525 109.225) (width 0.25) (layer "F.Cu") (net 1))
 (segment (start 152.7844 90.275) (end 153.305 90.275) (width 0.25) (layer "F.Cu") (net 1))
 (segment (start 154.491444 96.7) (end 154.491444 90.791444) (width 0.25) (layer "F.Cu") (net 1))
 (segment (start 158.14 96.56) (end 160.5 94.2) (width 0.25) (layer "F.Cu") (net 1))
 (segment (start 148.3 107.3) (end 151.511444 107.3) (width 0.25) (layer "F.Cu") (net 1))
 (segment (start 147 111) (end 148.3 109.7) (width 0.25) (layer "F.Cu") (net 1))
 (segment (start 175.4 94.1) (end 176.95 94.1) (width 0.25) (layer "F.Cu") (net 1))
 (segment (start 148.3 109.7) (end 148.3 107.3) (width 0.25) (layer "F.Cu") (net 1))
 (segment (start 154.491444 105.171444) (end 154.491444 104.32) (width 0.25) (layer "F.Cu") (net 1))
 (segment (start 151.511444 107.3) (end 154.491444 104.32) (width 0.25) (layer "F.Cu") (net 1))
 (segment (start 139.3 111) (end 147 111) (width 0.25) (layer "F.Cu") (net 1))
 (segment (start 144.25 97) (end 151.6 97) (width 0.25) (layer "F.Cu") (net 1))
 (segment (start 151.6 97) (end 151.9 96.7) (width 0.25) (layer "F.Cu") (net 1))
 (segment (start 148.8236 86.3142) (end 152.7844 90.275) (width 0.25) (layer "F.Cu") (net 1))
 (segment (start 153.975 90.275) (end 153.305 90.275) (width 0.25) (layer "F.Cu") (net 1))
 (segment (start 155.6 106.28) (end 154.491444 105.171444) (width 0.25) (layer "F.Cu") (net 1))
 (via (at 160.5 94.2) (size 0.8) (drill 0.4) (layers "F.Cu" "B.Cu") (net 1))
 (via (at 175.4 94.1) (size 0.8) (drill 0.4) (layers "F.Cu" "B.Cu") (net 1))
 (segment (start 160.5 94.2) (end 160.6 94.1) (width 0.25) (layer "B.Cu") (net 1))
 (segment (start 160.6 94.1) (end 175.4 94.1) (width 0.25) (layer "B.Cu") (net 1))
 (segment (start 133.6 91.82) (end 133.6 91) (width 0.25) (layer "F.Cu") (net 11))
 (segment (start 143 94.25) (end 143 98.5) (width 0.25) (layer "F.Cu") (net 11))
 (segment (start 133.6 91.82) (end 133.72 91.7) (width 0.25) (layer "F.Cu") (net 11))
 (segment (start 142.95 91.7) (end 144.25 93) (width 0.25) (layer "F.Cu") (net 11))
 (segment (start 152.7 98.5) (end 153.305 97.895) (width 0.25) (layer "F.Cu") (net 11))
 (segment (start 133.72 91.7) (end 142.95 91.7) (width 0.25) (layer "F.Cu") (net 11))
 (segment (start 127.525 97.895) (end 133.6 91.82) (width 0.25) (layer "F.Cu") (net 11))
 (segment (start 144.25 93) (end 143 94.25) (width 0.25) (layer "F.Cu") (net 11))
 (segment (start 143 98.5) (end 152.7 98.5) (width 0.25) (layer "F.Cu") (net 11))
 (segment (start 133.6 91) (end 133.5836 90.9836) (width 0.25) (layer "F.Cu") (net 11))
 (segment (start 133.5836 90.9836) (end 133.5836 86.3142) (width 0.25) (layer "F.Cu") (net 11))
 (segment (start 125.888557 86.579243) (end 127.3678 85.1) (width 0.25) (layer "F.Cu") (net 12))
 (segment (start 144.25 91) (end 142.05 88.8) (width 0.25) (layer "F.Cu") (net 12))
 (segment (start 127.3678 85.1) (end 129.8294 85.1) (width 0.25) (layer "F.Cu") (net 12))
 (segment (start 142.05 88.8) (end 135.3 88.8) (width 0.25) (layer "F.Cu") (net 12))
 (segment (start 149.635 100.435) (end 149 99.8) (width 0.25) (layer "F.Cu") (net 12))
 (segment (start 153.305 100.435) (end 149.635 100.435) (width 0.25) (layer "F.Cu") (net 12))
 (segment (start 127.525 100.435) (end 125.888557 98.798557) (width 0.25) (layer "F.Cu") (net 12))
 (segment (start 145.7 92) (end 145.25 92) (width 0.25) (layer "F.Cu") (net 12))
 (segment (start 125.888557 98.798557) (end 125.888557 86.579243) (width 0.25) (layer "F.Cu") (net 12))
 (segment (start 131.1 88.8) (end 131.0436 88.7436) (width 0.25) (layer "F.Cu") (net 12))
 (segment (start 145.25 92) (end 144.25 91) (width 0.25) (layer "F.Cu") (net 12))
 (segment (start 129.8294 85.1) (end 131.0436 86.3142) (width 0.25) (layer "F.Cu") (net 12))
 (segment (start 130.9508 86.3142) (end 131.0436 86.3142) (width 0.25) (layer "F.Cu") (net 12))
 (segment (start 131.0436 88.7436) (end 131.0436 86.3142) (width 0.25) (layer "F.Cu") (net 12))
 (via (at 131.1 88.8) (size 0.8) (drill 0.4) (layers "F.Cu" "B.Cu") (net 12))
 (via (at 149 99.8) (size 0.8) (drill 0.4) (layers "F.Cu" "B.Cu") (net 12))
 (via (at 145.7 92) (size 0.8) (drill 0.4) (layers "F.Cu" "B.Cu") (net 12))
 (via (at 135.3 88.8) (size 0.8) (drill 0.4) (layers "F.Cu" "B.Cu") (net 12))
 (segment (start 149 95.3) (end 145.7 92) (width 0.25) (layer "B.Cu") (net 12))
 (segment (start 135.3 88.8) (end 131.1 88.8) (width 0.25) (layer "B.Cu") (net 12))
 (segment (start 149 99.8) (end 149 95.3) (width 0.25) (layer "B.Cu") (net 12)))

